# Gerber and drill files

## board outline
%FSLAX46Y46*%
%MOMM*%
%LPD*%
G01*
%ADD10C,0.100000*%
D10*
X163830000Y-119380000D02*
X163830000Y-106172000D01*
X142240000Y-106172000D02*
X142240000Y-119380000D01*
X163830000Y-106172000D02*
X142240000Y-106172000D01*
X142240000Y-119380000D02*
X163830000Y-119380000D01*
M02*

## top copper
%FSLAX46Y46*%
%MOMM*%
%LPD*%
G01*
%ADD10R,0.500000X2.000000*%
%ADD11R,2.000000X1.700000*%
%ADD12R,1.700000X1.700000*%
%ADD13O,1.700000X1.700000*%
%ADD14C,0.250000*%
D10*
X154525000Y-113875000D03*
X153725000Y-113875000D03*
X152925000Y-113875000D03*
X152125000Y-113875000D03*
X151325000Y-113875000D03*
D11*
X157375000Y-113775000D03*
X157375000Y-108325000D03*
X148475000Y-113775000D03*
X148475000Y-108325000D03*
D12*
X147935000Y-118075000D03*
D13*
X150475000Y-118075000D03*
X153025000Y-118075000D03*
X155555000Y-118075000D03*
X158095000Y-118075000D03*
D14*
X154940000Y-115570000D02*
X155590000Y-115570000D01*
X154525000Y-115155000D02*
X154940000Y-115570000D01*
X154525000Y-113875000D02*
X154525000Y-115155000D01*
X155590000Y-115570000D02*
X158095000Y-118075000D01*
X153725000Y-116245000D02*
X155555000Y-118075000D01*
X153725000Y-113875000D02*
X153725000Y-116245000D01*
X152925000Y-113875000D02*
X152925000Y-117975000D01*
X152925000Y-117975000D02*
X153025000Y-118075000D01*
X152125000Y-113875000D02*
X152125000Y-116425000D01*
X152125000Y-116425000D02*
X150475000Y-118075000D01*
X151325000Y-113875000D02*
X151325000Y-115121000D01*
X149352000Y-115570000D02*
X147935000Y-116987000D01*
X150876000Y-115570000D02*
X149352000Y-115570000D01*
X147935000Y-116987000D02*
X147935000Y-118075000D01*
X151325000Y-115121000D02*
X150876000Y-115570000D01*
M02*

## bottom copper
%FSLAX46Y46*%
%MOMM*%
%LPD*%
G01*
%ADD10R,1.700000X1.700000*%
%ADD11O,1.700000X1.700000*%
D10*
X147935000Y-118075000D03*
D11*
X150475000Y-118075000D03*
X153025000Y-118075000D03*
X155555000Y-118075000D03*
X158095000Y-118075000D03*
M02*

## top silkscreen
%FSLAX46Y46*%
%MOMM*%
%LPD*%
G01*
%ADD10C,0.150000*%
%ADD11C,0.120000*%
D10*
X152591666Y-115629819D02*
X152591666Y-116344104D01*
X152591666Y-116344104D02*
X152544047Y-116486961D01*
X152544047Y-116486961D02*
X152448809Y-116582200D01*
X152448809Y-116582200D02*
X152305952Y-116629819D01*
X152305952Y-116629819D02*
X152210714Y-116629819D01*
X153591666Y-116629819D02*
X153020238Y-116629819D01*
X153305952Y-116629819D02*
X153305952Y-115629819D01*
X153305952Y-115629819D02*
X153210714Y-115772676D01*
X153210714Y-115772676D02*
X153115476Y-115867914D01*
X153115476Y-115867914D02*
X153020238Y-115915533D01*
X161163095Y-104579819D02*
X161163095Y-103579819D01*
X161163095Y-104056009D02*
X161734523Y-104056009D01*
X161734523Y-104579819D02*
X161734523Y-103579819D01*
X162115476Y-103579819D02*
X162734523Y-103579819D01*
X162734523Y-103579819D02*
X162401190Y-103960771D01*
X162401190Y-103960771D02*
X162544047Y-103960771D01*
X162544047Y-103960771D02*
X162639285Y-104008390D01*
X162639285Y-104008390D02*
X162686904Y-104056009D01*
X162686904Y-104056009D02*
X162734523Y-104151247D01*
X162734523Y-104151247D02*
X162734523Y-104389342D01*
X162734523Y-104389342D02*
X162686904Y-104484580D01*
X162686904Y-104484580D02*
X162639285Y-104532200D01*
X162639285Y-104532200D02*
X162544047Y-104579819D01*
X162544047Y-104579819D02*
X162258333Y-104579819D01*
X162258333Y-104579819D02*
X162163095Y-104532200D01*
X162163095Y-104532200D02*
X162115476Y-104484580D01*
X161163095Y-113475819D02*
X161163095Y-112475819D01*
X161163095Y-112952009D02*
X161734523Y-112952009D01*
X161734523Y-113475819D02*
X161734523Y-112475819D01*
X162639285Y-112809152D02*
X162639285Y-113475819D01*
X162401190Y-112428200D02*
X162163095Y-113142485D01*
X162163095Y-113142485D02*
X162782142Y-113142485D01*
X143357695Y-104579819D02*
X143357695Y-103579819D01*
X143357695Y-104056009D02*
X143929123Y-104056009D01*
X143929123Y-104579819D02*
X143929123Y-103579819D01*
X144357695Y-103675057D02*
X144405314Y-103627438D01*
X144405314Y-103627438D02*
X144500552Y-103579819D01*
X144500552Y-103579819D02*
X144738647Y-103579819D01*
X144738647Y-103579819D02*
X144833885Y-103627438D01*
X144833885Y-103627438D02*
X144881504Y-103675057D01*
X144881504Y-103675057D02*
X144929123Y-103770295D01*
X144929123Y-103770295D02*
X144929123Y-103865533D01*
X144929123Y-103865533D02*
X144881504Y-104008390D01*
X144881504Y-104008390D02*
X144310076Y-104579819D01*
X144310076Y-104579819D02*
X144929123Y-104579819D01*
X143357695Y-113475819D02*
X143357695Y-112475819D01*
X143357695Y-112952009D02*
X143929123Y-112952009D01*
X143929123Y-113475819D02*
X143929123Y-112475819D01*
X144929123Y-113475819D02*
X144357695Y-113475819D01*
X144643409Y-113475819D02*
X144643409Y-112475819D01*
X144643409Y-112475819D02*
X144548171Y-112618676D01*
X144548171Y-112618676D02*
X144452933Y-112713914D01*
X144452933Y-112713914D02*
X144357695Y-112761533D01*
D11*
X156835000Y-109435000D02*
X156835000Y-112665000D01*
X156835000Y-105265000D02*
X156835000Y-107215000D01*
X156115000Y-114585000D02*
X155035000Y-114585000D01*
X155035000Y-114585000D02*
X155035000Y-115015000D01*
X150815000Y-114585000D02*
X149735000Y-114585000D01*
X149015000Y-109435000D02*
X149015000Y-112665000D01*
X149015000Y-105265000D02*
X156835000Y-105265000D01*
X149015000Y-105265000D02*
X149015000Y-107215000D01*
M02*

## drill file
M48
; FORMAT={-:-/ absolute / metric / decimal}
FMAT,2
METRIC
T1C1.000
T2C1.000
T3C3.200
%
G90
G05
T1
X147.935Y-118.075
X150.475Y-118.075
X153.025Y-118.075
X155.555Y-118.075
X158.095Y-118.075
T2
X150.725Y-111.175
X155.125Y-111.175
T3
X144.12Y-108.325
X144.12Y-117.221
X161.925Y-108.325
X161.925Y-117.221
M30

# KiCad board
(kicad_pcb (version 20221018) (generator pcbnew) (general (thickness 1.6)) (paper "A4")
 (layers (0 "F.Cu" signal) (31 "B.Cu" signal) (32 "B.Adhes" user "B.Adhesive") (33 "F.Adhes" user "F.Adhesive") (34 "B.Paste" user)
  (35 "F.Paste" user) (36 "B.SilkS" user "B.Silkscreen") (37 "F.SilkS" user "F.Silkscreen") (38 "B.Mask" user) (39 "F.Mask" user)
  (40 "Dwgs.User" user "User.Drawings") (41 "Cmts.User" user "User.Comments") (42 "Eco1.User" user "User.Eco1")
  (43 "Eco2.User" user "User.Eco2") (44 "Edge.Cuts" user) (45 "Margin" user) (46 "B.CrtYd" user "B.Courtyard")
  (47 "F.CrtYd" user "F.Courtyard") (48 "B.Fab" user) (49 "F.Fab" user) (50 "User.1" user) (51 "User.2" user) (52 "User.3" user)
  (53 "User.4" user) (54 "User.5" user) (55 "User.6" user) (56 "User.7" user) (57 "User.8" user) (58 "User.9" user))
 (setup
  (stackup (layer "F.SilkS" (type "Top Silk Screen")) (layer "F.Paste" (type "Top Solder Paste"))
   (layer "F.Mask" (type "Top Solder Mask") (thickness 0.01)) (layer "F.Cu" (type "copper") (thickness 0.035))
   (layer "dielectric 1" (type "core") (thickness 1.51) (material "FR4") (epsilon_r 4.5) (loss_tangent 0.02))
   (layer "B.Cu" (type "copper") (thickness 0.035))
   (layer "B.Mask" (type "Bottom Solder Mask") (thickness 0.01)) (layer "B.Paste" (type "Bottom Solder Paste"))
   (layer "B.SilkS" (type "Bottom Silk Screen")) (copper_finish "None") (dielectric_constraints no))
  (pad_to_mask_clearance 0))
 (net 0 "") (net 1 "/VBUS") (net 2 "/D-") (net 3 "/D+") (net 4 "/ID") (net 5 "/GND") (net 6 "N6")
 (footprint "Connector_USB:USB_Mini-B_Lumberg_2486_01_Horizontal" (layer "F.Cu") (at 152.925 111.175 180)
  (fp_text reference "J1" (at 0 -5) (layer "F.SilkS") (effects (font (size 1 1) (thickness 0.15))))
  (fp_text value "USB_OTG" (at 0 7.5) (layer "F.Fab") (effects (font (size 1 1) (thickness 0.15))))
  (fp_line (start -3.91 1.74) (end -3.91 -1.49) (stroke (width 0.12) (type solid)) (layer "F.SilkS"))
  (fp_line (start -3.91 5.91) (end -3.91 3.96) (stroke (width 0.12) (type solid)) (layer "F.SilkS"))
  (fp_line (start -3.19 -3.41) (end -2.11 -3.41) (stroke (width 0.12) (type solid)) (layer "F.SilkS"))
  (fp_line (start -2.11 -3.41) (end -2.11 -3.84) (stroke (width 0.12) (type solid)) (layer "F.SilkS"))
  (fp_line (start 2.11 -3.41) (end 3.19 -3.41) (stroke (width 0.12) (type solid)) (layer "F.SilkS"))
  (fp_line (start 3.91 1.74) (end 3.91 -1.49) (stroke (width 0.12) (type solid)) (layer "F.SilkS"))
  (fp_line (start 3.91 5.91) (end -3.91 5.91) (stroke (width 0.12) (type solid)) (layer "F.SilkS"))
  (fp_line (start 3.91 5.91) (end 3.91 3.96) (stroke (width 0.12) (type solid)) (layer "F.SilkS"))
  (pad "" np_thru_hole circle (at -2.2 0 180) (size 1 1) (drill 1) (layers "*.Cu" "*.Mask"))
  (pad "" np_thru_hole circle (at 2.2 0 180) (size 1 1) (drill 1) (layers "*.Cu" "*.Mask"))
  (pad "1" smd rect (at -1.6 -2.7 180) (size 0.5 2) (layers "F.Cu" "F.Paste" "F.Mask") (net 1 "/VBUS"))
  (pad "2" smd rect (at -0.8 -2.7 180) (size 0.5 2) (layers "F.Cu" "F.Paste" "F.Mask") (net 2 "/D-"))
  (pad "3" smd rect (at 0 -2.7 180) (size 0.5 2) (layers "F.Cu" "F.Paste" "F.Mask") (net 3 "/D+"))
  (pad "4" smd rect (at 0.8 -2.7 180) (size 0.5 2) (layers "F.Cu" "F.Paste" "F.Mask") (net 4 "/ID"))
  (pad "5" smd rect (at 1.6 -2.7 180) (size 0.5 2) (layers "F.Cu" "F.Paste" "F.Mask") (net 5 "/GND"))
  (pad "6" smd rect (at -4.45 -2.6 180) (size 2 1.7) (layers "F.Cu" "F.Paste" "F.Mask") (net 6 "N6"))
  (pad "6" smd rect (at -4.45 2.85 180) (size 2 1.7) (layers "F.Cu" "F.Paste" "F.Mask") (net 6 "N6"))
  (pad "6" smd rect (at 4.45 -2.6 180) (size 2 1.7) (layers "F.Cu" "F.Paste" "F.Mask") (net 6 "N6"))
  (pad "6" smd rect (at 4.45 2.85 180) (size 2 1.7) (layers "F.Cu" "F.Paste" "F.Mask") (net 6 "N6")))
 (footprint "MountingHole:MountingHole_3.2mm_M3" (layer "F.Cu") (at 161.925 108.325)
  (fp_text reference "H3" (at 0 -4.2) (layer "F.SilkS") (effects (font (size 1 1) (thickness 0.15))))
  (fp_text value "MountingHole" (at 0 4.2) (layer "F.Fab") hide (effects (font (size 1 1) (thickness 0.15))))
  (pad "" np_thru_hole circle (at 0 0) (size 3.2 3.2) (drill 3.2) (layers "*.Cu" "*.Mask")))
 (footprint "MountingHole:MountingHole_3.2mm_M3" (layer "F.Cu") (at 161.925 117.221)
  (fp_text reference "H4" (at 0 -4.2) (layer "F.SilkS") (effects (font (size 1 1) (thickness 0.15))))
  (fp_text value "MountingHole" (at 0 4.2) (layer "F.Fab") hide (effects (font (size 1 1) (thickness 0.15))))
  (pad "" np_thru_hole circle (at 0 0) (size 3.2 3.2) (drill 3.2) (layers "*.Cu" "*.Mask")))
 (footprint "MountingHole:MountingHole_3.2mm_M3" (layer "F.Cu") (at 144.1196 108.325)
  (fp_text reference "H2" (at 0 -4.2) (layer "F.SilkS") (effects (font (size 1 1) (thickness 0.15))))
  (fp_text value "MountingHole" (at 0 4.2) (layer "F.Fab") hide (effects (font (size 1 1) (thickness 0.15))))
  (pad "" np_thru_hole circle (at 0 0) (size 3.2 3.2) (drill 3.2) (layers "*.Cu" "*.Mask")))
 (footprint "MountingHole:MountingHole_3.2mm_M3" (layer "F.Cu") (at 144.1196 117.221)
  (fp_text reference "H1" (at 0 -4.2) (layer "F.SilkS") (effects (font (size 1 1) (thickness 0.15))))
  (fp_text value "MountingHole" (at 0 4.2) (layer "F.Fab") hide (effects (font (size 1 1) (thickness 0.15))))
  (pad "" np_thru_hole circle (at 0 0) (size 3.2 3.2) (drill 3.2) (layers "*.Cu" "*.Mask")))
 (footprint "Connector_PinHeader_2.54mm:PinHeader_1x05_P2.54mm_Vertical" (layer "B.Cu") (at 147.935 118.075 -90)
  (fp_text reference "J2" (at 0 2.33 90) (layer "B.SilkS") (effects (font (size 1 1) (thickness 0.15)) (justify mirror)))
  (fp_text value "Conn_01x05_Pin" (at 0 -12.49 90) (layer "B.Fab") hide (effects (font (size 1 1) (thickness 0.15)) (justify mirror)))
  (pad "1" thru_hole rect (at 0 0 270) (size 1.7 1.7) (drill 1) (layers "*.Cu" "*.Mask") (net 5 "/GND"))
  (pad "2" thru_hole oval (at 0 -2.54 270) (size 1.7 1.7) (drill 1) (layers "*.Cu" "*.Mask") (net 4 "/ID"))
  (pad "3" thru_hole oval (at 0 -5.09 270) (size 1.7 1.7) (drill 1) (layers "*.Cu" "*.Mask") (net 3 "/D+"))
  (pad "4" thru_hole oval (at 0 -7.62 270) (size 1.7 1.7) (drill 1) (layers "*.Cu" "*.Mask") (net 2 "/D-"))
  (pad "5" thru_hole oval (at 0 -10.16 270) (size 1.7 1.7) (drill 1) (layers "*.Cu" "*.Mask") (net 1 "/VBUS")))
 (gr_line (start 163.83 119.38) (end 163.83 106.172) (stroke (width 0.1) (type default)) (layer "Edge.Cuts"))
 (gr_line (start 142.24 106.172) (end 142.24 119.38) (stroke (width 0.1) (type default)) (layer "Edge.Cuts"))
 (gr_line (start 163.83 106.172) (end 142.24 106.172) (stroke (width 0.1) (type default)) (layer "Edge.Cuts"))
 (gr_line (start 142.24 119.38) (end 163.83 119.38) (stroke (width 0.1) (type default)) (layer "Edge.Cuts"))
 (segment (start 154.94 115.57) (end 155.59 115.57) (width 0.25) (layer "F.Cu") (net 1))
 (segment (start 154.525 115.155) (end 154.94 115.57) (width 0.25) (layer "F.Cu") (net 1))
 (segment (start 154.525 113.875) (end 154.525 115.155) (width 0.25) (layer "F.Cu") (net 1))
 (segment (start 155.59 115.57) (end 158.095 118.075) (width 0.25) (layer "F.Cu") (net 1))
 (segment (start 153.725 116.245) (end 155.555 118.075) (width 0.25) (layer "F.Cu") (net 2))
 (segment (start 153.725 113.875) (end 153.725 116.245) (width 0.25) (layer "F.Cu") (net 2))
 (segment (start 152.925 113.875) (end 152.925 117.975) (width 0.25) (layer "F.Cu") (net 3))
 (segment (start 152.925 117.975) (end 153.025 118.075) (width 0.25) (layer "F.Cu") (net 3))
 (segment (start 152.125 113.875) (end 152.125 116.425) (width 0.25) (layer "F.Cu") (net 4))
 (segment (start 152.125 116.425) (end 150.475 118.075) (width 0.25) (layer "F.Cu") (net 4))
 (segment (start 151.325 113.875) (end 151.325 115.121) (width 0.25) (layer "F.Cu") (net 5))
 (segment (start 149.352 115.57) (end 147.935 116.987) (width 0.25) (layer "F.Cu") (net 5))
 (segment (start 150.876 115.57) (end 149.352 115.57) (width 0.25) (layer "F.Cu") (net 5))
 (segment (start 147.935 116.987) (end 147.935 118.075) (width 0.25) (layer "F.Cu") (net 5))
 (segment (start 151.325 115.121) (end 150.876 115.57) (width 0.25) (layer "F.Cu") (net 5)))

